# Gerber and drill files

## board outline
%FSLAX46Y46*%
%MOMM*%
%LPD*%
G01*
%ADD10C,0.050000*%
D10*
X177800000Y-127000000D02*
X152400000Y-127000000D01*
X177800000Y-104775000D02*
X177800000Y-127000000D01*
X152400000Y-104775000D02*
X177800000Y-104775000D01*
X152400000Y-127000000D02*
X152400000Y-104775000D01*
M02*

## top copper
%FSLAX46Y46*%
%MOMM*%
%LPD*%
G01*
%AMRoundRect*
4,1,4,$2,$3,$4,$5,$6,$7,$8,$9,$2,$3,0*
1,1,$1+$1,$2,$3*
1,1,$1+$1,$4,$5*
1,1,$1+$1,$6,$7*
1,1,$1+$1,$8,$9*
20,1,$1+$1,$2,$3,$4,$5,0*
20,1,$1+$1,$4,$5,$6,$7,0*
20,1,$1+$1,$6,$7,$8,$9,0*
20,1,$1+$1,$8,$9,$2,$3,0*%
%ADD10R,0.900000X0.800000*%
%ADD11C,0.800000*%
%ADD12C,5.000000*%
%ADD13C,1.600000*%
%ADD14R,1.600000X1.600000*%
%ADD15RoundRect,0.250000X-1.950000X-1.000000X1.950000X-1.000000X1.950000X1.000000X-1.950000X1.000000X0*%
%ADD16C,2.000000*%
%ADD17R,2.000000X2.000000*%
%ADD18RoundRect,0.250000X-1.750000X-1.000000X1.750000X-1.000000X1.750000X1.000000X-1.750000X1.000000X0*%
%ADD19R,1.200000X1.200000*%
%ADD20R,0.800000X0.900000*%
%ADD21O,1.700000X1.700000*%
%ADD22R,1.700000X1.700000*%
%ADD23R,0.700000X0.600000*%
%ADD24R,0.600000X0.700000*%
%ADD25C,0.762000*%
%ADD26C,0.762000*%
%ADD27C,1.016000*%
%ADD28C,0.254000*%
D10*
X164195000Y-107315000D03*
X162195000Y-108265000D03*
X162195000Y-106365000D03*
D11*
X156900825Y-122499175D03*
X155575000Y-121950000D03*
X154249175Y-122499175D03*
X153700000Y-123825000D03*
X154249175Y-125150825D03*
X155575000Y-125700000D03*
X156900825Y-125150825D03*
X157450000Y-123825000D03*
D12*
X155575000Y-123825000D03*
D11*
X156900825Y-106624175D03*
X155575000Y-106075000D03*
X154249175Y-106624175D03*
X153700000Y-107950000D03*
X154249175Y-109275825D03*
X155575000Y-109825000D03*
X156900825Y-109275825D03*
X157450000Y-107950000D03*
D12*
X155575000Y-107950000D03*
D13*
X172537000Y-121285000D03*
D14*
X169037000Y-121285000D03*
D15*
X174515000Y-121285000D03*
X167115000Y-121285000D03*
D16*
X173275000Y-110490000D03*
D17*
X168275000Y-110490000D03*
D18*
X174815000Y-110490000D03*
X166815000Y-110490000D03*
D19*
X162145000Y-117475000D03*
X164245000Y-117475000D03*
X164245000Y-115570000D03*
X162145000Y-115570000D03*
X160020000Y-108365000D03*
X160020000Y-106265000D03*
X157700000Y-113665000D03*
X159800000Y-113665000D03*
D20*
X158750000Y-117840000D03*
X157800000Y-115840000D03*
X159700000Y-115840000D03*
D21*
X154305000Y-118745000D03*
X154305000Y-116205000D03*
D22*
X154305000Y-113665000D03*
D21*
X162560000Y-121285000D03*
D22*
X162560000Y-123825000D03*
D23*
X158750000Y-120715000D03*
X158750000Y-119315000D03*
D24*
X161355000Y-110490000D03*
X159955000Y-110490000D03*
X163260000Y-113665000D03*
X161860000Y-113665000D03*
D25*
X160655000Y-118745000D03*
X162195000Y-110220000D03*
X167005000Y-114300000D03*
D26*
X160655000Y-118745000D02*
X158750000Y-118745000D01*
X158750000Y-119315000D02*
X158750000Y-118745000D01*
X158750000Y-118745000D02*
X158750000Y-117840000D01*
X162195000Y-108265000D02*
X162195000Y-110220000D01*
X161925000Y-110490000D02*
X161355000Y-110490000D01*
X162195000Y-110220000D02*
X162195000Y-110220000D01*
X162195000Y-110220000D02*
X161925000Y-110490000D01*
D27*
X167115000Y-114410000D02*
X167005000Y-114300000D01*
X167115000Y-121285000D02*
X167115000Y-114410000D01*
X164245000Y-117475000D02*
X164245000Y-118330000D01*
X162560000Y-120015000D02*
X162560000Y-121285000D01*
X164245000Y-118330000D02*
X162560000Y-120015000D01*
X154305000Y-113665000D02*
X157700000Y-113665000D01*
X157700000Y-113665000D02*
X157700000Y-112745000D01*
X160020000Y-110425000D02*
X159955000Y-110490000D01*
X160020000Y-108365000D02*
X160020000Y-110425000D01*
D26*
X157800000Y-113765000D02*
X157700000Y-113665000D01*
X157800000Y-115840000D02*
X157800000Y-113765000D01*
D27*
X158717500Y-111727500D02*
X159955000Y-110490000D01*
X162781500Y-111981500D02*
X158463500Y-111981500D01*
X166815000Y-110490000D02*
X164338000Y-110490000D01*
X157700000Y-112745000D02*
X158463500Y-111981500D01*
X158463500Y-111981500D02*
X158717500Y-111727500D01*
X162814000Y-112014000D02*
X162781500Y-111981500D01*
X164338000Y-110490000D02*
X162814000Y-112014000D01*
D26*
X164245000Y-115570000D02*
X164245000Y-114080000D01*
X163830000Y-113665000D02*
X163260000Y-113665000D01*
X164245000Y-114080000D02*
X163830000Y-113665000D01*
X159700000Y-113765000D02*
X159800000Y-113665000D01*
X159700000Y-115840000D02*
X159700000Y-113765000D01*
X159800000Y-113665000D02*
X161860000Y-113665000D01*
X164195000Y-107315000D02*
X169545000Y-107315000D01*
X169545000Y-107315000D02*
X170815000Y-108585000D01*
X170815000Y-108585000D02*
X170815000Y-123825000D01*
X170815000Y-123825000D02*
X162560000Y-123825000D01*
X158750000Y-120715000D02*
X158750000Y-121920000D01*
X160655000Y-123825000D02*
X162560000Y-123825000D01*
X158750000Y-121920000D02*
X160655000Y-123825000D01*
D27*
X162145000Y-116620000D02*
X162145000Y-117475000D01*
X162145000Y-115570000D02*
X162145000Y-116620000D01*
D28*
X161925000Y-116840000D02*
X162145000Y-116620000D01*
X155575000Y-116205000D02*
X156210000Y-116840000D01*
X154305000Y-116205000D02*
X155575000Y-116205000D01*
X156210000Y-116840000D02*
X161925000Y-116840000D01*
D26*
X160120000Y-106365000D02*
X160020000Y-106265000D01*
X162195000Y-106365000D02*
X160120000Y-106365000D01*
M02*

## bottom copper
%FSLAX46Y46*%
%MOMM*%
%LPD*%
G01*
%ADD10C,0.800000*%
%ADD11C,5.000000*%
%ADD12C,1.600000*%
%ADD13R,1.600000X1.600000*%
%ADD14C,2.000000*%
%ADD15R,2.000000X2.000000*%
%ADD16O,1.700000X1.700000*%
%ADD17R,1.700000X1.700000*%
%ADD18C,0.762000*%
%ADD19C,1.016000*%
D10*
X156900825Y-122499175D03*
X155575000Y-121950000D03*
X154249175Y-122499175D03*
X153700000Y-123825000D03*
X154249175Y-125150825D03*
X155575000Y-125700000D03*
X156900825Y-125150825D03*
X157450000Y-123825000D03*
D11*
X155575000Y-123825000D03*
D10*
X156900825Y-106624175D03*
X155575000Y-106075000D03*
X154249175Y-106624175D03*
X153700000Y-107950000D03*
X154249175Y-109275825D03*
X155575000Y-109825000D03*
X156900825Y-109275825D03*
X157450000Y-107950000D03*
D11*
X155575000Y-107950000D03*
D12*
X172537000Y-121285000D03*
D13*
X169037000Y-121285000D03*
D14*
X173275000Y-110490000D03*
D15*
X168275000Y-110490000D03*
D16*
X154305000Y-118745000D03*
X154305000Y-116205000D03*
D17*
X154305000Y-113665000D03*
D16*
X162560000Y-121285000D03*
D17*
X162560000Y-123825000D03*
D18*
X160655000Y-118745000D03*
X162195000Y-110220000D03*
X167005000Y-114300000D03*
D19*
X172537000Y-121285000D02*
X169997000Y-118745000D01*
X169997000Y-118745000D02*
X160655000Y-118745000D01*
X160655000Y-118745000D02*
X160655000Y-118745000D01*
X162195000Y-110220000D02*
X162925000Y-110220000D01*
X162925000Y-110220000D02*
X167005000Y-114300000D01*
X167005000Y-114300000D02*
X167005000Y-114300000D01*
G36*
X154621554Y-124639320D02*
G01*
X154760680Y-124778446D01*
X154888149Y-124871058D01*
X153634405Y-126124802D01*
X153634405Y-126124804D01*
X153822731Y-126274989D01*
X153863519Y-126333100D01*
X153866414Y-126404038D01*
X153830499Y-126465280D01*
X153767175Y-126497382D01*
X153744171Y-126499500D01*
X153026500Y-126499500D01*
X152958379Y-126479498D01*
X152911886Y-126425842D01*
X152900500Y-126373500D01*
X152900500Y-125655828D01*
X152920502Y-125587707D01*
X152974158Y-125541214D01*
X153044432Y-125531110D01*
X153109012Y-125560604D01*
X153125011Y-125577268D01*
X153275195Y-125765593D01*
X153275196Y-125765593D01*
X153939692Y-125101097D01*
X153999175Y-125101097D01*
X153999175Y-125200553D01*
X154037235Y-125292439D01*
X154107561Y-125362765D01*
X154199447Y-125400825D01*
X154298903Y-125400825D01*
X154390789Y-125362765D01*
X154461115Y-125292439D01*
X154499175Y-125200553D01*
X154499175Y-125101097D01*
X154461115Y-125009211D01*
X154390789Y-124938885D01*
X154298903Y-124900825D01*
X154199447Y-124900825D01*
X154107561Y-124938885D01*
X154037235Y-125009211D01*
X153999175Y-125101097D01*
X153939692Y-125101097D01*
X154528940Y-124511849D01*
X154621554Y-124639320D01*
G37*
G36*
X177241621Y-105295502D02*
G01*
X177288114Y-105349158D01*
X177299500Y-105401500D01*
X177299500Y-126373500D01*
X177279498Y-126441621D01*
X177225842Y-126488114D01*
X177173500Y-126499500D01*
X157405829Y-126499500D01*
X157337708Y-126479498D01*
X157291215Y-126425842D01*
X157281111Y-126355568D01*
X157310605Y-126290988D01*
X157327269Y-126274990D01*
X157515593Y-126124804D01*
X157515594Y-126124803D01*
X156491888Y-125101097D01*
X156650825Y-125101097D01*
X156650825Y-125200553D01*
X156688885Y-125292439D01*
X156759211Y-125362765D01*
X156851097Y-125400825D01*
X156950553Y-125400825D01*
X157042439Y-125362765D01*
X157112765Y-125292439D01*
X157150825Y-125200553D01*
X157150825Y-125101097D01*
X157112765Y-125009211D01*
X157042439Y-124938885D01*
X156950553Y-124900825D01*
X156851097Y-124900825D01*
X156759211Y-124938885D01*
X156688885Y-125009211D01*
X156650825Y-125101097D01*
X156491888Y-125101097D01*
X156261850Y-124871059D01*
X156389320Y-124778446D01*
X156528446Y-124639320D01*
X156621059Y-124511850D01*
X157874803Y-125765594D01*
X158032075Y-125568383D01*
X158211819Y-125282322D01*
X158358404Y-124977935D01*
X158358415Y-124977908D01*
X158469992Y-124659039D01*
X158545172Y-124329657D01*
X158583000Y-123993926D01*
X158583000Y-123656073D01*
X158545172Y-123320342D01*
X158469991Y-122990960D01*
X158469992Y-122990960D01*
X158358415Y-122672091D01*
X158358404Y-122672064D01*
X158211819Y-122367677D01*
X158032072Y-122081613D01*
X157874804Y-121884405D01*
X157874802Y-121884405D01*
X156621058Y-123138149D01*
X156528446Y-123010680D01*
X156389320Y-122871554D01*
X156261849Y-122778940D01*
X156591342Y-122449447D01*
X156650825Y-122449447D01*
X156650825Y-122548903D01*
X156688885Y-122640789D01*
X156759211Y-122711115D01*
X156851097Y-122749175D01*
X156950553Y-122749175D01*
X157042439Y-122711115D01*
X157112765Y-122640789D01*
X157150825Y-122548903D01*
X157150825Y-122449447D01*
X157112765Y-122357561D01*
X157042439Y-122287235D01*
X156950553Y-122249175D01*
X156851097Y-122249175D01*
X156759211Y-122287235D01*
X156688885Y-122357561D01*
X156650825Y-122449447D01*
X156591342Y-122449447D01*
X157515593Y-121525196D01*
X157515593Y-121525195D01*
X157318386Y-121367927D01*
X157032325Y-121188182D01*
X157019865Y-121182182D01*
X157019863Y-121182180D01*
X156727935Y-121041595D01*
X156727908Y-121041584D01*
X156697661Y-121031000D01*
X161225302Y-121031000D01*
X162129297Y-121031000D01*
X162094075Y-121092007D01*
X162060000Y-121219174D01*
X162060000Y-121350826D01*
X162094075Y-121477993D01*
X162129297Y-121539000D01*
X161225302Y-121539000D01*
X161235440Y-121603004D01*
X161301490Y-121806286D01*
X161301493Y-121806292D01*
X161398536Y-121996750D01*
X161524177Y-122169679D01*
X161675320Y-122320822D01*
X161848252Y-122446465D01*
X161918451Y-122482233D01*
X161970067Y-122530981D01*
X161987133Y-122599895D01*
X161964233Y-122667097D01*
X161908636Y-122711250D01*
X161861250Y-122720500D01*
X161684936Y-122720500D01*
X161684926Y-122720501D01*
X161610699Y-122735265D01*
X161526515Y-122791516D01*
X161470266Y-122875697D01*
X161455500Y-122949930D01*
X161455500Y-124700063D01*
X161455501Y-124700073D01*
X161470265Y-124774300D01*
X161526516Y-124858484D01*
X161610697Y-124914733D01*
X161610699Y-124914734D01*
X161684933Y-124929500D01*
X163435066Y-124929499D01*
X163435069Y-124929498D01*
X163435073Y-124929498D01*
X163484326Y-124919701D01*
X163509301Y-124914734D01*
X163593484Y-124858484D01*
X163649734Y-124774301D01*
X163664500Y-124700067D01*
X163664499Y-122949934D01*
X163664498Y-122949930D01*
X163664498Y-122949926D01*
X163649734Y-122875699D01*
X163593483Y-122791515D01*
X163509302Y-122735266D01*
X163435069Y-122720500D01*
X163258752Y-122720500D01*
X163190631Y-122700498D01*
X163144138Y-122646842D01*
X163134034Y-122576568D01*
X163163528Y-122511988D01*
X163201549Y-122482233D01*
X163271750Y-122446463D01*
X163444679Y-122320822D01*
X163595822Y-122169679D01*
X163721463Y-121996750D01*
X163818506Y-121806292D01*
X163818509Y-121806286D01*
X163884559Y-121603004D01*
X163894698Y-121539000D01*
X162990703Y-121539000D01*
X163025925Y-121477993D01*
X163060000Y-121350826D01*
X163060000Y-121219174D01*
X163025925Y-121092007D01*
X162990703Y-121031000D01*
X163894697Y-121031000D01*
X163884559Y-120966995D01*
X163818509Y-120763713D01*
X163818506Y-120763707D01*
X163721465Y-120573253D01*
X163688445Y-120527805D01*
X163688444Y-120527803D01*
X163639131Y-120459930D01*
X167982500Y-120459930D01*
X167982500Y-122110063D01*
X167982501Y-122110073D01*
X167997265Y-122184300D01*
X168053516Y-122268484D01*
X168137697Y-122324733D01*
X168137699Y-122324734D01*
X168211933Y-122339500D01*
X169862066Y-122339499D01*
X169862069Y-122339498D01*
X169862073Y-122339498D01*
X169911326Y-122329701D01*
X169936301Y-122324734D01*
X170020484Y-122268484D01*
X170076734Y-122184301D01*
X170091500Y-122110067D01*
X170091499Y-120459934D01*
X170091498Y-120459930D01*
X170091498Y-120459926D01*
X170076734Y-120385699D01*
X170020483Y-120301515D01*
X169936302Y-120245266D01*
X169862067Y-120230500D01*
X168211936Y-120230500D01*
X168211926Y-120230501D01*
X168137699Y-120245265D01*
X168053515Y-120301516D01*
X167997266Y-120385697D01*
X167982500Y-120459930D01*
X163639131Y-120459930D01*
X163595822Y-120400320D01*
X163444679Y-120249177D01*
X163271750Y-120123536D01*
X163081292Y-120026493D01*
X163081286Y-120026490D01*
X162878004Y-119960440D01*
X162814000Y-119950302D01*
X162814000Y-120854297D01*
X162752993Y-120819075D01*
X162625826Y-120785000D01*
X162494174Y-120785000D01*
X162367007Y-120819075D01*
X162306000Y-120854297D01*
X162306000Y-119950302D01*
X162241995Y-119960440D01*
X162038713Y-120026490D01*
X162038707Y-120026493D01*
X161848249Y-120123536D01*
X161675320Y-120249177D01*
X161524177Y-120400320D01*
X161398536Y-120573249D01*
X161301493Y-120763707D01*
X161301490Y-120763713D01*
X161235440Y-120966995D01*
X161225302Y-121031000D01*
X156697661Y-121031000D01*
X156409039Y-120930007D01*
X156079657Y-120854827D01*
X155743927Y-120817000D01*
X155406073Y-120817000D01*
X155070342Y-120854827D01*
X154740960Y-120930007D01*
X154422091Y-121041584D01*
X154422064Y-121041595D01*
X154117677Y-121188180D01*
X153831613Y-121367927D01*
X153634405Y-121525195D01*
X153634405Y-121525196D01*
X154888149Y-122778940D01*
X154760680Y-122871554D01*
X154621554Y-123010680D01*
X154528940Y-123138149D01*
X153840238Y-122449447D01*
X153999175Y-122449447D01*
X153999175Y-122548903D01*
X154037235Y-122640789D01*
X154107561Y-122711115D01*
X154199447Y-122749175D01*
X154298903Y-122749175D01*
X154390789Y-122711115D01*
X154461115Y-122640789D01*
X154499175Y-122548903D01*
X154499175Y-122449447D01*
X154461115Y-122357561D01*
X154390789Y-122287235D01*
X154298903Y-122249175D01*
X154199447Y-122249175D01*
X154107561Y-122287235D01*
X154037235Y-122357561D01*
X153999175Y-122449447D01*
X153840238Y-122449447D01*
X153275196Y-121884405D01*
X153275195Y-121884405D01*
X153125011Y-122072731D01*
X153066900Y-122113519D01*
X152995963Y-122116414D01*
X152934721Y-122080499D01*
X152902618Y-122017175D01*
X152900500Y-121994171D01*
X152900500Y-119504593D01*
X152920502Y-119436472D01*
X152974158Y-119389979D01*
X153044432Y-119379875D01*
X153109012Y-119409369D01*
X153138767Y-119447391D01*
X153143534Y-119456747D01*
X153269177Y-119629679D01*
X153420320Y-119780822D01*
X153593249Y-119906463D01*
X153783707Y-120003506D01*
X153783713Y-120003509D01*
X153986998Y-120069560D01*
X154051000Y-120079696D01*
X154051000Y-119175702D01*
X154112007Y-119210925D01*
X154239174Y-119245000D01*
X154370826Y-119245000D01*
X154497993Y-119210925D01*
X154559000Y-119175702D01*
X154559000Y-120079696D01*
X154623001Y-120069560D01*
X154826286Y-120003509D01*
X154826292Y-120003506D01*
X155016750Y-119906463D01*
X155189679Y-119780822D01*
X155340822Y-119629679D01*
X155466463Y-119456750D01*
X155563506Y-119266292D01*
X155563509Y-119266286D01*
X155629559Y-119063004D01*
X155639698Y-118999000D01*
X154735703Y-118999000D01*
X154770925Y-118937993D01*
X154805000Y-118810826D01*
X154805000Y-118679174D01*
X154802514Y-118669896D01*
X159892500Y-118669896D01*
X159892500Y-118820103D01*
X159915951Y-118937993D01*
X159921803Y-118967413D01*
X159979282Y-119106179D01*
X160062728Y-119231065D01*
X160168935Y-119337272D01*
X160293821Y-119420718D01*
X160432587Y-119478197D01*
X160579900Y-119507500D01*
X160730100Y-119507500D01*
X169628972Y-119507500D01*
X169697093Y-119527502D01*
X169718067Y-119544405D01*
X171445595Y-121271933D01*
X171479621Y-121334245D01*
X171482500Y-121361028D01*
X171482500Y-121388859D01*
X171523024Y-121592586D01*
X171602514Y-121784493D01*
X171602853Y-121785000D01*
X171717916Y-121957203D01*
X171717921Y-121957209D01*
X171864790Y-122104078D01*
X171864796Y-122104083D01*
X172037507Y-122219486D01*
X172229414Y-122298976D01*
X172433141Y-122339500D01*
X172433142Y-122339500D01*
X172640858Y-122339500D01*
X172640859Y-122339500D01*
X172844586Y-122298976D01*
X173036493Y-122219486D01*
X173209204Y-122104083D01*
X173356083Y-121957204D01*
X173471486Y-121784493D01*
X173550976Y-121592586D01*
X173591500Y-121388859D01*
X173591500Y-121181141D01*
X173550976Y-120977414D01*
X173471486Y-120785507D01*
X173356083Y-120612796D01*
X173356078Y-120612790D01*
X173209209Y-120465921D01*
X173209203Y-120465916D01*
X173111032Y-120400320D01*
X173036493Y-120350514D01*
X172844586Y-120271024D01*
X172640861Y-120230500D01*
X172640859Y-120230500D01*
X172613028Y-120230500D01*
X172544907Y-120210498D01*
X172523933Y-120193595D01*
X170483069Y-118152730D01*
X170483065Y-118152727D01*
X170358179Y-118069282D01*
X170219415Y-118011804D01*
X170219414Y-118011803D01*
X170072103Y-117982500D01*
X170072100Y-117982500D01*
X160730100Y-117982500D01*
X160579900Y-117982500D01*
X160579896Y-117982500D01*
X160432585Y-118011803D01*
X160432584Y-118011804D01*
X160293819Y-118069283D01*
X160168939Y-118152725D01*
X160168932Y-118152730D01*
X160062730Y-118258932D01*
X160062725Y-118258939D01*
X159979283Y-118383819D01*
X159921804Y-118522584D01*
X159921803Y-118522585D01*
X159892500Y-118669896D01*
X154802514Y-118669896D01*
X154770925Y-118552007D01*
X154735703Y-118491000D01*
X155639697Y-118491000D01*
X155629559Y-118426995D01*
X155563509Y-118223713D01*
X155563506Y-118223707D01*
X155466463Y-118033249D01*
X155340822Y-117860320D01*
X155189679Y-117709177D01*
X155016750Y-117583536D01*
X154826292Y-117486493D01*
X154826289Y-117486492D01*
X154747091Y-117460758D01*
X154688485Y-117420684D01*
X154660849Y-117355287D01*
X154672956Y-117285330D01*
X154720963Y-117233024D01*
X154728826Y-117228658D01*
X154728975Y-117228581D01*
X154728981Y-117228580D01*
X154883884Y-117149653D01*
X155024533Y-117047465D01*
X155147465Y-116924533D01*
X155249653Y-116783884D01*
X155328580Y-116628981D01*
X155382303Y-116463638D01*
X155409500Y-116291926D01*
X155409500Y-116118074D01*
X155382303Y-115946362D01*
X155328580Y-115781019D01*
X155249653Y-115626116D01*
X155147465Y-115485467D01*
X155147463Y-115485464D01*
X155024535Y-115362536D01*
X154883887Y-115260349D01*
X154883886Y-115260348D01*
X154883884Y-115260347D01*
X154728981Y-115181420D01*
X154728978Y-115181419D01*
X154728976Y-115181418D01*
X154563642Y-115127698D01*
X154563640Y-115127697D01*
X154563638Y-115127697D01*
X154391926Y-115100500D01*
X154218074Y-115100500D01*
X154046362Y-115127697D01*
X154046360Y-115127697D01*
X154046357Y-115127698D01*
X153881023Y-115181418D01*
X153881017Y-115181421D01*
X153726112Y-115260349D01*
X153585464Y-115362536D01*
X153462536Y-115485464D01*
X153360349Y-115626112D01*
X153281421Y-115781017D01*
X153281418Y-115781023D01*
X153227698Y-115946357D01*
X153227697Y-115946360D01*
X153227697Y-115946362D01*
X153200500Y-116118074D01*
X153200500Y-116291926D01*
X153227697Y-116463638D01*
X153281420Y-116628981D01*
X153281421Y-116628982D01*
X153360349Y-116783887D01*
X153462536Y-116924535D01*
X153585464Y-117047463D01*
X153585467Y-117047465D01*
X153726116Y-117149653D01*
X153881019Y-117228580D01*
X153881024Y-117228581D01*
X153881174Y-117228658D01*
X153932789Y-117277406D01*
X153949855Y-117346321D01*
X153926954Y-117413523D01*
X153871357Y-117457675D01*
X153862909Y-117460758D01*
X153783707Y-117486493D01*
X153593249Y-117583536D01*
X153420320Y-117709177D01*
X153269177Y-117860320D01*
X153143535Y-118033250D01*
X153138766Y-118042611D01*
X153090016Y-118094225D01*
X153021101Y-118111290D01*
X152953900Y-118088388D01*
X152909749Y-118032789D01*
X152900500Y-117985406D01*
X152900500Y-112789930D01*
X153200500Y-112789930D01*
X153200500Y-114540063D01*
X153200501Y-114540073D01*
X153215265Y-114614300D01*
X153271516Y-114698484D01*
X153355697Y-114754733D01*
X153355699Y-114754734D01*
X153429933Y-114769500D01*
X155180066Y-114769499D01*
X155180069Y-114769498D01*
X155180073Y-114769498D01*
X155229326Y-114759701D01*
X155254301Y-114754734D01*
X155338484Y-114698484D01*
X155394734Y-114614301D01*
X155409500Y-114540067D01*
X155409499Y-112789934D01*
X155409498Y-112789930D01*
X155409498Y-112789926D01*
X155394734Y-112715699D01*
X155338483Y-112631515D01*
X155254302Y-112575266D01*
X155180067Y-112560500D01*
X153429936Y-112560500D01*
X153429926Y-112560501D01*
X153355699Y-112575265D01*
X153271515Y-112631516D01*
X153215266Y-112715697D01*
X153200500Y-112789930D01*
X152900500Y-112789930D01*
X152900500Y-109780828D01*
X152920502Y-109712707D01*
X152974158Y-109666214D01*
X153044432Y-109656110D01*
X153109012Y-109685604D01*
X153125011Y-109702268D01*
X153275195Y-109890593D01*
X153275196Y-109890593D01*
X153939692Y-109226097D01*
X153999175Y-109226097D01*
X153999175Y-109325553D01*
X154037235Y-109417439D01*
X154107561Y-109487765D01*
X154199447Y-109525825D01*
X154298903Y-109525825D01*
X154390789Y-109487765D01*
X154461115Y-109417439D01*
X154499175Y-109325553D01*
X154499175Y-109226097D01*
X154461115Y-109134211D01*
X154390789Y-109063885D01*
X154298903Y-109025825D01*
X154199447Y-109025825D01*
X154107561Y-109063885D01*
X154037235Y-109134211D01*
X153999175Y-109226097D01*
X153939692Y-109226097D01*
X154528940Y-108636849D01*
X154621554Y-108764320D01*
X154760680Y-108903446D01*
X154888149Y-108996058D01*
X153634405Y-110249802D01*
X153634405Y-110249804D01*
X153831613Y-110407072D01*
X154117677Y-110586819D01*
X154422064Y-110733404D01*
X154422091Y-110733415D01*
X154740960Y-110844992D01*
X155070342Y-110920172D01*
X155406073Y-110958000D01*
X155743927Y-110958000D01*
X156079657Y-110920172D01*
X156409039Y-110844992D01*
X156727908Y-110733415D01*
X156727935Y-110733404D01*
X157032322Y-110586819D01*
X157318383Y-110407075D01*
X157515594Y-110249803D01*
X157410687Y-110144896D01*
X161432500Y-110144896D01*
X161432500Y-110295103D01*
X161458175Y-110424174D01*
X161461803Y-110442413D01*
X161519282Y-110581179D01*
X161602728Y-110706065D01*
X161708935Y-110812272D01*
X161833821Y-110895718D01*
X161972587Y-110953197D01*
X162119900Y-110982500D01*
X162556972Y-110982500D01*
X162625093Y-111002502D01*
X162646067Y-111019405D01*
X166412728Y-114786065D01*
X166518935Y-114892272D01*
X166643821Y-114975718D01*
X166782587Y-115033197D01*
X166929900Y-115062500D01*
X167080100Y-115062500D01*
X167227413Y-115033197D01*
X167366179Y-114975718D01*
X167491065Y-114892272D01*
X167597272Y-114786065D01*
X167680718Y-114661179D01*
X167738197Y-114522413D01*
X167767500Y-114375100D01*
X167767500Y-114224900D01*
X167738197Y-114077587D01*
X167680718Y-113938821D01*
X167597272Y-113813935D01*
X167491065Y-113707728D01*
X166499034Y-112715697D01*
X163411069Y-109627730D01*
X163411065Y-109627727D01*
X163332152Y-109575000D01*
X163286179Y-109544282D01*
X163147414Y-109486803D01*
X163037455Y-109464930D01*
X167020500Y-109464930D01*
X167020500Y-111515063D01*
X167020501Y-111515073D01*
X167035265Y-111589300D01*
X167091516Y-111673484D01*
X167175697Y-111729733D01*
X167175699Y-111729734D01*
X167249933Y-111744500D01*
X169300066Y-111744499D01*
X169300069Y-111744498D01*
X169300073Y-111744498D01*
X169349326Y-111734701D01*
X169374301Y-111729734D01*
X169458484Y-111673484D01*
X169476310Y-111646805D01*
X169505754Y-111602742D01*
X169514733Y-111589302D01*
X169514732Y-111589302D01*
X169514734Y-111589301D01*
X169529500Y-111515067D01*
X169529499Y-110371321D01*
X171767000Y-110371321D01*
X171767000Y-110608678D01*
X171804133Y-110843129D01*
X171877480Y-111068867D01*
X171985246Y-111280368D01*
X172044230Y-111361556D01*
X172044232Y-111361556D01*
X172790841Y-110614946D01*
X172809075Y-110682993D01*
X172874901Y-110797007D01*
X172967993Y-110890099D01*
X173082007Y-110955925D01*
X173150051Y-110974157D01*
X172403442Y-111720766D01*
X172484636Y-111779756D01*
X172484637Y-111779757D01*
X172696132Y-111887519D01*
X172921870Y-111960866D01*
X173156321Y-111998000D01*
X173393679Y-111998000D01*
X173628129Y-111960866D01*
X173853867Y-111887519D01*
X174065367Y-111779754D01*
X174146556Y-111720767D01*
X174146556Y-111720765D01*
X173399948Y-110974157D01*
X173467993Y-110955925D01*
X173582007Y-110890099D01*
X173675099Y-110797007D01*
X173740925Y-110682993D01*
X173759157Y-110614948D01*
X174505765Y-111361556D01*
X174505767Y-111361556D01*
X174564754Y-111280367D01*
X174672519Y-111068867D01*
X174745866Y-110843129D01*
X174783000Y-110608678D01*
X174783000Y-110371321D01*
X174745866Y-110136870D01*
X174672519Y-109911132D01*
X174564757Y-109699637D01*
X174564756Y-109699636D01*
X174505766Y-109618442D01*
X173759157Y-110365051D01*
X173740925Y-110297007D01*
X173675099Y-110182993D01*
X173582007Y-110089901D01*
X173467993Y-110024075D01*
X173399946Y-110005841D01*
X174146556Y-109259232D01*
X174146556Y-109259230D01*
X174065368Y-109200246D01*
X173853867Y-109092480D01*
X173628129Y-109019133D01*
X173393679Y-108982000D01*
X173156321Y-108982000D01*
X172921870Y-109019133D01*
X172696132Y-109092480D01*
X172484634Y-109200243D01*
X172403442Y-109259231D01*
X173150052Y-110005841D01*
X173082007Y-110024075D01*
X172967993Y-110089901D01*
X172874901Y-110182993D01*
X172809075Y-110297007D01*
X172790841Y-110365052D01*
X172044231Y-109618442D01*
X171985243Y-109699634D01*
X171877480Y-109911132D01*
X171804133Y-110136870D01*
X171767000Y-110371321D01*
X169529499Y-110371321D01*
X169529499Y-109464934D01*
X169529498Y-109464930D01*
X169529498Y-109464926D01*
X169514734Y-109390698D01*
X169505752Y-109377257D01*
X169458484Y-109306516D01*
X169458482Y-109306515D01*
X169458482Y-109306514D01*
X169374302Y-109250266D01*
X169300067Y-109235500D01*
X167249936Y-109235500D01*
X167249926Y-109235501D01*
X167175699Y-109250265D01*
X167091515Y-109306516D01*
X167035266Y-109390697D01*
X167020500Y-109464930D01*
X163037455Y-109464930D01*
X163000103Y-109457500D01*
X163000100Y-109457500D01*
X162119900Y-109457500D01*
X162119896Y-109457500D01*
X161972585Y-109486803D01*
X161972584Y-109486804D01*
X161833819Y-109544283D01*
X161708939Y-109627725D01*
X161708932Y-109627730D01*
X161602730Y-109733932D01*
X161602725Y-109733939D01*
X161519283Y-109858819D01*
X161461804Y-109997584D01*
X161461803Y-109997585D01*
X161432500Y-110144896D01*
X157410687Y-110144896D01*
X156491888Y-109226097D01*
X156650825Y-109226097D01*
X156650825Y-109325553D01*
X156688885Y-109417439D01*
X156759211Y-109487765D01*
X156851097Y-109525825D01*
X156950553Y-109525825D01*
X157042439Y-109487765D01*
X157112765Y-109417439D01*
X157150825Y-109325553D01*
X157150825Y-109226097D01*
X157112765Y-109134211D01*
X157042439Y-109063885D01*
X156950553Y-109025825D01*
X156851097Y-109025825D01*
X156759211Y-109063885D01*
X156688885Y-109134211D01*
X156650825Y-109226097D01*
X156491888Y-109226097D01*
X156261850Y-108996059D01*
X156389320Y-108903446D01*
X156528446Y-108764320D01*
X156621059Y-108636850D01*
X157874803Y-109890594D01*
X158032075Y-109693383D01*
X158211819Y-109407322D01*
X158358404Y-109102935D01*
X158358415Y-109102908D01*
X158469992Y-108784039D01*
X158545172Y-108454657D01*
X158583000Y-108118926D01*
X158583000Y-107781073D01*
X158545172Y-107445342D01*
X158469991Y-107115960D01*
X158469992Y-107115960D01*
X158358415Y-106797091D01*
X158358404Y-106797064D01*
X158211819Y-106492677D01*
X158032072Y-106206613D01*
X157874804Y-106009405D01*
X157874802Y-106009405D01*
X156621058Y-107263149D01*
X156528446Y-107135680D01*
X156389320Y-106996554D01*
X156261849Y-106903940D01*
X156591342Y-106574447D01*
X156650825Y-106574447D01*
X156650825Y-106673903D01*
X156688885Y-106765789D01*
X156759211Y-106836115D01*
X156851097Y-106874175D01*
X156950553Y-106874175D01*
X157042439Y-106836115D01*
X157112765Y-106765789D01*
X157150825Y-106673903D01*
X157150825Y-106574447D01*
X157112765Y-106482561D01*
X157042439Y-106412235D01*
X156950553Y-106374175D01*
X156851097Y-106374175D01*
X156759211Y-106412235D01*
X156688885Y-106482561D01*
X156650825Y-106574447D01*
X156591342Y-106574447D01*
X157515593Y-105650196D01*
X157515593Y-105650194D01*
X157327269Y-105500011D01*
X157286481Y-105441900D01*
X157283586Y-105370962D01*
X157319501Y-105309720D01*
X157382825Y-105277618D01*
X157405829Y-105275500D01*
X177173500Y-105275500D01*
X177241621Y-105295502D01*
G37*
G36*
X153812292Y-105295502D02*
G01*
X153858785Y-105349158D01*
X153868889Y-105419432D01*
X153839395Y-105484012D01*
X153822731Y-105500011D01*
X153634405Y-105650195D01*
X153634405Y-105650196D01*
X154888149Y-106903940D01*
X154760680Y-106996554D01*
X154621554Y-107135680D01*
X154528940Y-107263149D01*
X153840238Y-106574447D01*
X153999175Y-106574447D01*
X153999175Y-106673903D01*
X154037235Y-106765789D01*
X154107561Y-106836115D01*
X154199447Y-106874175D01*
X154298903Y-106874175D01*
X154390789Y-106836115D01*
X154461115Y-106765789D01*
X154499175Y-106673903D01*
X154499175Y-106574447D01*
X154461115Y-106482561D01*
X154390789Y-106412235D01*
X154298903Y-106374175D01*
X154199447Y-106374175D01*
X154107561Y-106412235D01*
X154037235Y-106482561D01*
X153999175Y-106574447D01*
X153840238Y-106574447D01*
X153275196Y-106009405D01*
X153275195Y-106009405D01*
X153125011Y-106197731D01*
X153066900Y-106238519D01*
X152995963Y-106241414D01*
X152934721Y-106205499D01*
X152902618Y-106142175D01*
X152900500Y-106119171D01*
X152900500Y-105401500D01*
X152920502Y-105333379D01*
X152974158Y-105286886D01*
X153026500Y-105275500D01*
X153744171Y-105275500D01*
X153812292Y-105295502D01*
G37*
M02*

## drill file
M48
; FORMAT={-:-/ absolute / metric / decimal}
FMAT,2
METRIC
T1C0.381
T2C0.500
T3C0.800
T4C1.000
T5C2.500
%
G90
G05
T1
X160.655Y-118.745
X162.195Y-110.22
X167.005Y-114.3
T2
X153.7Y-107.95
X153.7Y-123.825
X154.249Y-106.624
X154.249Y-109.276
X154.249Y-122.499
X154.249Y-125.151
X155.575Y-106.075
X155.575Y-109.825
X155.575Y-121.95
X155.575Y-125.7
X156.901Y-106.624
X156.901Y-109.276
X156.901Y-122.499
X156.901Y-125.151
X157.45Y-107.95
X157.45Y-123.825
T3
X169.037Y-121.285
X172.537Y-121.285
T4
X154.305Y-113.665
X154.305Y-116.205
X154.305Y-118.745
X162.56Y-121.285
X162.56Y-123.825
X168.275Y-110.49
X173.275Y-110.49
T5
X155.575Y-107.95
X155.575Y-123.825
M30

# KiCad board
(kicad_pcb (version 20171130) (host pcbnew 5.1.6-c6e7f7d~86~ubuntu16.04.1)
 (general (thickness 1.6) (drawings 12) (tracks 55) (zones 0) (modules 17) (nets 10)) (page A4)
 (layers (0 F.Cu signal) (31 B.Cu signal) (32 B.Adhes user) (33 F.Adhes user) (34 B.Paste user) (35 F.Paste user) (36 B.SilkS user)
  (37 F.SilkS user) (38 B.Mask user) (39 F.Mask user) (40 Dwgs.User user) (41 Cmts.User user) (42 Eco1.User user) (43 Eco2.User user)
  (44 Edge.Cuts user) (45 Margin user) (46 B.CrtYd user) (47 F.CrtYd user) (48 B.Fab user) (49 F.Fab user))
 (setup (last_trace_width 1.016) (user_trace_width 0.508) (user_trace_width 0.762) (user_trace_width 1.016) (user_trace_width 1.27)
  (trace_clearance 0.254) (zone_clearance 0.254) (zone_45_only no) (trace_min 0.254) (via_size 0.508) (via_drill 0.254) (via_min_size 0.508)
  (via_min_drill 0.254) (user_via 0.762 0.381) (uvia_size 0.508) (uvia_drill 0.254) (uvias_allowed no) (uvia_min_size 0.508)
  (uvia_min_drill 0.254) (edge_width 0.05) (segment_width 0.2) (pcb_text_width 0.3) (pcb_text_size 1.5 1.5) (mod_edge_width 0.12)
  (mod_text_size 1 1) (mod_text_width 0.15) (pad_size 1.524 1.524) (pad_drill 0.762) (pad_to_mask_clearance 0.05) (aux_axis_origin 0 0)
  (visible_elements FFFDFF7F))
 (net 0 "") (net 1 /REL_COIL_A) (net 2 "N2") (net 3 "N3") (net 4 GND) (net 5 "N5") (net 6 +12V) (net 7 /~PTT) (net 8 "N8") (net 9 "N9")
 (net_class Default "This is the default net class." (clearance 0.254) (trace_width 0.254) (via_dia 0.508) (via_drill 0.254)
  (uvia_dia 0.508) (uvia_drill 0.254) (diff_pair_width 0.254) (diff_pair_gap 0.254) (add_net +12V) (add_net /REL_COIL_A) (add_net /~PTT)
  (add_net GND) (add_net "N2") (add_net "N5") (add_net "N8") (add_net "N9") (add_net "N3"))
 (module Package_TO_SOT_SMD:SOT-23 (layer F.Cu) (at 163.195 107.315)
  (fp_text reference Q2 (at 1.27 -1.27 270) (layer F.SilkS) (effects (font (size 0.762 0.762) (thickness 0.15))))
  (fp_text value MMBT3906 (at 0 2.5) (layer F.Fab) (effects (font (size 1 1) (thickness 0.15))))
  (pad 3 smd rect (at 1 0) (size 0.9 0.8) (layers F.Cu F.Paste F.Mask) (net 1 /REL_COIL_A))
  (pad 2 smd rect (at -1 0.95) (size 0.9 0.8) (layers F.Cu F.Paste F.Mask) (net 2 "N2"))
  (pad 1 smd rect (at -1 -0.95) (size 0.9 0.8) (layers F.Cu F.Paste F.Mask) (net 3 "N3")))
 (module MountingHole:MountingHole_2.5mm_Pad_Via (layer F.Cu) (at 155.575 123.825)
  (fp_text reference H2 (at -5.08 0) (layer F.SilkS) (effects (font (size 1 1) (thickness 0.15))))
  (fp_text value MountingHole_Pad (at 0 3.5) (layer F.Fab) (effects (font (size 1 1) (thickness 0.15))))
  (pad 1 thru_hole circle (at 1.325825 -1.325825) (size 0.8 0.8) (drill 0.5) (layers *.Cu *.Mask) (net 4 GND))
  (pad 1 thru_hole circle (at 0 -1.875) (size 0.8 0.8) (drill 0.5) (layers *.Cu *.Mask) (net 4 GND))
  (pad 1 thru_hole circle (at -1.325825 -1.325825) (size 0.8 0.8) (drill 0.5) (layers *.Cu *.Mask) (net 4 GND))
  (pad 1 thru_hole circle (at -1.875 0) (size 0.8 0.8) (drill 0.5) (layers *.Cu *.Mask) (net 4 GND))
  (pad 1 thru_hole circle (at -1.325825 1.325825) (size 0.8 0.8) (drill 0.5) (layers *.Cu *.Mask) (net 4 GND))
  (pad 1 thru_hole circle (at 0 1.875) (size 0.8 0.8) (drill 0.5) (layers *.Cu *.Mask) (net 4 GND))
  (pad 1 thru_hole circle (at 1.325825 1.325825) (size 0.8 0.8) (drill 0.5) (layers *.Cu *.Mask) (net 4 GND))
  (pad 1 thru_hole circle (at 1.875 0) (size 0.8 0.8) (drill 0.5) (layers *.Cu *.Mask) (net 4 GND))
  (pad 1 thru_hole circle (at 0 0) (size 5 5) (drill 2.5) (layers *.Cu *.Mask) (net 4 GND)))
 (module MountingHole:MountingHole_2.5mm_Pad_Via (layer F.Cu) (at 155.575 107.95)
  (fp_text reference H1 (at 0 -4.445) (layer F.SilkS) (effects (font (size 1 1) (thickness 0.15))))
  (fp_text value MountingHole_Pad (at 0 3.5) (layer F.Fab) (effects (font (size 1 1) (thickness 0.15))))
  (pad 1 thru_hole circle (at 1.325825 -1.325825) (size 0.8 0.8) (drill 0.5) (layers *.Cu *.Mask) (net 4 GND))
  (pad 1 thru_hole circle (at 0 -1.875) (size 0.8 0.8) (drill 0.5) (layers *.Cu *.Mask) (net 4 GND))
  (pad 1 thru_hole circle (at -1.325825 -1.325825) (size 0.8 0.8) (drill 0.5) (layers *.Cu *.Mask) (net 4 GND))
  (pad 1 thru_hole circle (at -1.875 0) (size 0.8 0.8) (drill 0.5) (layers *.Cu *.Mask) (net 4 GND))
  (pad 1 thru_hole circle (at -1.325825 1.325825) (size 0.8 0.8) (drill 0.5) (layers *.Cu *.Mask) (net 4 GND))
  (pad 1 thru_hole circle (at 0 1.875) (size 0.8 0.8) (drill 0.5) (layers *.Cu *.Mask) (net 4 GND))
  (pad 1 thru_hole circle (at 1.325825 1.325825) (size 0.8 0.8) (drill 0.5) (layers *.Cu *.Mask) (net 4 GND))
  (pad 1 thru_hole circle (at 1.875 0) (size 0.8 0.8) (drill 0.5) (layers *.Cu *.Mask) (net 4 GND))
  (pad 1 thru_hole circle (at 0 0) (size 5 5) (drill 2.5) (layers *.Cu *.Mask) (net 4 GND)))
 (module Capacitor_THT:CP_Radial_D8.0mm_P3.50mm (layer F.Cu) (at 169.037 121.285)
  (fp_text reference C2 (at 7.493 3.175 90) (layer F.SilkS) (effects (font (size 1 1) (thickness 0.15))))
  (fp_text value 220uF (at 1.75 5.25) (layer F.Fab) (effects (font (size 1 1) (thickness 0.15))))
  (pad 2 thru_hole circle (at 3.5 0) (size 1.6 1.6) (drill 0.8) (layers *.Cu *.Mask) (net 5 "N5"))
  (pad 1 thru_hole rect (at 0 0) (size 1.6 1.6) (drill 0.8) (layers *.Cu *.Mask) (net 2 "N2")))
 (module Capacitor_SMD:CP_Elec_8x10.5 (layer F.Cu) (at 170.815 121.285)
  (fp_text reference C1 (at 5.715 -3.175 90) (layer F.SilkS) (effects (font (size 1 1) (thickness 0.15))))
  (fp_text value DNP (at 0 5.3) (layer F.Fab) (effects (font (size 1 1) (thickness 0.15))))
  (pad 2 smd roundrect (at 3.7 0) (size 4.4 2.5) (layers F.Cu F.Paste F.Mask) (roundrect_rratio 0.1) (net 5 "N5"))
  (pad 1 smd roundrect (at -3.7 0) (size 4.4 2.5) (layers F.Cu F.Paste F.Mask) (roundrect_rratio 0.1) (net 2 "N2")))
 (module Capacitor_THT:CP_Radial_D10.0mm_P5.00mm (layer F.Cu) (at 168.275 110.49)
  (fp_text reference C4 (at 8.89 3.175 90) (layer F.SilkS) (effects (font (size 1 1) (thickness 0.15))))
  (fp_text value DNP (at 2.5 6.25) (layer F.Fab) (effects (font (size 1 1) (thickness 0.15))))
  (pad 2 thru_hole circle (at 5 0) (size 2 2) (drill 1) (layers *.Cu *.Mask) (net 4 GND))
  (pad 1 thru_hole rect (at 0 0) (size 2 2) (drill 1) (layers *.Cu *.Mask) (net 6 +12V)))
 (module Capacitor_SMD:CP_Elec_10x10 (layer F.Cu) (at 170.815 110.49)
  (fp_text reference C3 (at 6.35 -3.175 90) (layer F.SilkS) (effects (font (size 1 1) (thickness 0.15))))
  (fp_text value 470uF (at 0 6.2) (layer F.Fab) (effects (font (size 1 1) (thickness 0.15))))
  (pad 2 smd roundrect (at 4 0) (size 4 2.5) (layers F.Cu F.Paste F.Mask) (roundrect_rratio 0.1) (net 4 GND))
  (pad 1 smd roundrect (at -4 0) (size 4 2.5) (layers F.Cu F.Paste F.Mask) (roundrect_rratio 0.1) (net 6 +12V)))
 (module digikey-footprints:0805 (layer F.Cu) (at 163.195 117.475)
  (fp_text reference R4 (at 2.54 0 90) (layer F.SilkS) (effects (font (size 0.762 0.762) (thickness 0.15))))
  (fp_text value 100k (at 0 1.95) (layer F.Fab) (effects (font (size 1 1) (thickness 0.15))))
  (pad 1 smd rect (at -1.05 0) (size 1.2 1.2) (layers F.Cu F.Paste F.Mask) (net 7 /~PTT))
  (pad 2 smd rect (at 1.05 0) (size 1.2 1.2) (layers F.Cu F.Paste F.Mask) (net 4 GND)))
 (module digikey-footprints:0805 (layer F.Cu) (at 163.195 115.57 180)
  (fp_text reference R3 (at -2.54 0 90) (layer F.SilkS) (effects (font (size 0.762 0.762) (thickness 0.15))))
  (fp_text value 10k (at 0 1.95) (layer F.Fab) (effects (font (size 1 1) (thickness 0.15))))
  (pad 1 smd rect (at -1.05 0 180) (size 1.2 1.2) (layers F.Cu F.Paste F.Mask) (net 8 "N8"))
  (pad 2 smd rect (at 1.05 0 180) (size 1.2 1.2) (layers F.Cu F.Paste F.Mask) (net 7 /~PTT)))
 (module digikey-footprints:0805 (layer F.Cu) (at 160.02 107.315 90)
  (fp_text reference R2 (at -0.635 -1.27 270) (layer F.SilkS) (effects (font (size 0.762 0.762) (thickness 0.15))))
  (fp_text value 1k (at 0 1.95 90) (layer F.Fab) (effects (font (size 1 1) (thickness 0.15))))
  (pad 1 smd rect (at -1.05 0 90) (size 1.2 1.2) (layers F.Cu F.Paste F.Mask) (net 6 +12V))
  (pad 2 smd rect (at 1.05 0 90) (size 1.2 1.2) (layers F.Cu F.Paste F.Mask) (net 3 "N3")))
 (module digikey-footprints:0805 (layer F.Cu) (at 158.75 113.665)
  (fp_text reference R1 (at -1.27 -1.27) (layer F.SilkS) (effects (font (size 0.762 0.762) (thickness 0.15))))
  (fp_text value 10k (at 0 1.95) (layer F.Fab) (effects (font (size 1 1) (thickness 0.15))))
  (pad 1 smd rect (at -1.05 0) (size 1.2 1.2) (layers F.Cu F.Paste F.Mask) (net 6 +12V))
  (pad 2 smd rect (at 1.05 0) (size 1.2 1.2) (layers F.Cu F.Paste F.Mask) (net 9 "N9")))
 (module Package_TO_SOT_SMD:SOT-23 (layer F.Cu) (at 158.75 116.84 270)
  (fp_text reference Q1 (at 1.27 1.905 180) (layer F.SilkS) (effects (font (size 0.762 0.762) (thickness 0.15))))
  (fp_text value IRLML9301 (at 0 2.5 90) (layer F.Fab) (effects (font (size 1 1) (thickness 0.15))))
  (pad 3 smd rect (at 1 0 270) (size 0.9 0.8) (layers F.Cu F.Paste F.Mask) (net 5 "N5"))
  (pad 2 smd rect (at -1 0.95 270) (size 0.9 0.8) (layers F.Cu F.Paste F.Mask) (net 6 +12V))
  (pad 1 smd rect (at -1 -0.95 270) (size 0.9 0.8) (layers F.Cu F.Paste F.Mask) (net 9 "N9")))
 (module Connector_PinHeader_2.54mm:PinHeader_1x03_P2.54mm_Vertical (layer F.Cu) (at 154.305 113.665)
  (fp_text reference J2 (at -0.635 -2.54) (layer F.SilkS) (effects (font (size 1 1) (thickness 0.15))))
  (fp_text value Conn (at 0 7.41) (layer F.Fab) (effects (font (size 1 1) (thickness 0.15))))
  (pad 3 thru_hole oval (at 0 5.08) (size 1.7 1.7) (drill 1) (layers *.Cu *.Mask) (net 4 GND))
  (pad 2 thru_hole oval (at 0 2.54) (size 1.7 1.7) (drill 1) (layers *.Cu *.Mask) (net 7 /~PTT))
  (pad 1 thru_hole rect (at 0 0) (size 1.7 1.7) (drill 1) (layers *.Cu *.Mask) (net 6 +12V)))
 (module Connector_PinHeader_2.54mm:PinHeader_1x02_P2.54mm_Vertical (layer F.Cu) (at 162.56 123.825 180)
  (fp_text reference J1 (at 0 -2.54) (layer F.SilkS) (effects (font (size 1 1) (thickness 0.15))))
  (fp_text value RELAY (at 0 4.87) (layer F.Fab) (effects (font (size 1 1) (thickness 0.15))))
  (pad 2 thru_hole oval (at 0 2.54 180) (size 1.7 1.7) (drill 1) (layers *.Cu *.Mask) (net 4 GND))
  (pad 1 thru_hole rect (at 0 0 180) (size 1.7 1.7) (drill 1) (layers *.Cu *.Mask) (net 1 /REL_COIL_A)))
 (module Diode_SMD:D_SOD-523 (layer F.Cu) (at 158.75 120.015 90)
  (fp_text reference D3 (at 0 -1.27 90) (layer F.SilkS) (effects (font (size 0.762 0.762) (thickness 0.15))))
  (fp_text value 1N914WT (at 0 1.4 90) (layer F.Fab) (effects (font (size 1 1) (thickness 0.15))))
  (pad 1 smd rect (at -0.7 0 270) (size 0.6 0.7) (layers F.Cu F.Paste F.Mask) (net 1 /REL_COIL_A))
  (pad 2 smd rect (at 0.7 0 270) (size 0.6 0.7) (layers F.Cu F.Paste F.Mask) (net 5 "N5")))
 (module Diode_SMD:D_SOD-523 (layer F.Cu) (at 160.655 110.49 180)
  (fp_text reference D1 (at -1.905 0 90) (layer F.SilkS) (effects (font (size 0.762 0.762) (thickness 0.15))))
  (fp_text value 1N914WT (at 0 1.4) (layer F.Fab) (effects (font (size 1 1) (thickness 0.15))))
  (pad 1 smd rect (at -0.7 0) (size 0.6 0.7) (layers F.Cu F.Paste F.Mask) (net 2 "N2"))
  (pad 2 smd rect (at 0.7 0) (size 0.6 0.7) (layers F.Cu F.Paste F.Mask) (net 6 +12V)))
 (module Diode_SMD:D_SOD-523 (layer F.Cu) (at 162.56 113.665 180)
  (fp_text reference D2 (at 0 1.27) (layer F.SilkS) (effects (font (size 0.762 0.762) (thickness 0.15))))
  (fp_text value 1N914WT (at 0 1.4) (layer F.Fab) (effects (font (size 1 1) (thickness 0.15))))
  (pad 1 smd rect (at -0.7 0) (size 0.6 0.7) (layers F.Cu F.Paste F.Mask) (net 8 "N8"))
  (pad 2 smd rect (at 0.7 0) (size 0.6 0.7) (layers F.Cu F.Paste F.Mask) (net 9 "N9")))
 (gr_line (start 177.8 127) (end 152.4 127) (layer Edge.Cuts) (width 0.05))
 (gr_line (start 177.8 104.775) (end 177.8 127) (layer Edge.Cuts) (width 0.05))
 (gr_line (start 152.4 104.775) (end 177.8 104.775) (layer Edge.Cuts) (width 0.05))
 (gr_line (start 152.4 127) (end 152.4 104.775) (layer Edge.Cuts) (width 0.05))
 (segment (start 172.537 121.285) (end 169.997 118.745) (width 1.016) (layer B.Cu) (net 5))
 (segment (start 169.997 118.745) (end 160.655 118.745) (width 1.016) (layer B.Cu) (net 5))
 (segment (start 160.655 118.745) (end 160.655 118.745) (width 1.016) (layer B.Cu) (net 5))
 (via (at 160.655 118.745) (size 0.762) (drill 0.381) (layers F.Cu B.Cu) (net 5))
 (segment (start 160.655 118.745) (end 158.75 118.745) (width 0.762) (layer F.Cu) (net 5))
 (segment (start 158.75 119.315) (end 158.75 118.745) (width 0.762) (layer F.Cu) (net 5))
 (segment (start 158.75 118.745) (end 158.75 117.84) (width 0.762) (layer F.Cu) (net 5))
 (segment (start 162.195 108.265) (end 162.195 110.22) (width 0.762) (layer F.Cu) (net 2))
 (segment (start 161.925 110.49) (end 161.355 110.49) (width 0.762) (layer F.Cu) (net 2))
 (segment (start 162.195 110.22) (end 162.195 110.22) (width 0.762) (layer F.Cu) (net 2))
 (segment (start 162.195 110.22) (end 161.925 110.49) (width 0.762) (layer F.Cu) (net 2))
 (via (at 162.195 110.22) (size 0.762) (drill 0.381) (layers F.Cu B.Cu) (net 2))
 (segment (start 162.195 110.22) (end 162.925 110.22) (width 1.016) (layer B.Cu) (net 2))
 (segment (start 162.925 110.22) (end 167.005 114.3) (width 1.016) (layer B.Cu) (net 2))
 (segment (start 167.005 114.3) (end 167.005 114.3) (width 1.016) (layer B.Cu) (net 2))
 (via (at 167.005 114.3) (size 0.762) (drill 0.381) (layers F.Cu B.Cu) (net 2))
 (segment (start 167.115 114.41) (end 167.005 114.3) (width 1.016) (layer F.Cu) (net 2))
 (segment (start 167.115 121.285) (end 167.115 114.41) (width 1.016) (layer F.Cu) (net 2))
 (segment (start 164.245 117.475) (end 164.245 118.33) (width 1.016) (layer F.Cu) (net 4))
 (segment (start 162.56 120.015) (end 162.56 121.285) (width 1.016) (layer F.Cu) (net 4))
 (segment (start 164.245 118.33) (end 162.56 120.015) (width 1.016) (layer F.Cu) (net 4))
 (segment (start 154.305 113.665) (end 157.7 113.665) (width 1.016) (layer F.Cu) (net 6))
 (segment (start 157.7 113.665) (end 157.7 112.745) (width 1.016) (layer F.Cu) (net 6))
 (segment (start 160.02 110.425) (end 159.955 110.49) (width 1.016) (layer F.Cu) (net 6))
 (segment (start 160.02 108.365) (end 160.02 110.425) (width 1.016) (layer F.Cu) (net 6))
 (segment (start 157.8 113.765) (end 157.7 113.665) (width 0.762) (layer F.Cu) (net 6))
 (segment (start 157.8 115.84) (end 157.8 113.765) (width 0.762) (layer F.Cu) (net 6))
 (segment (start 158.7175 111.7275) (end 159.955 110.49) (width 1.016) (layer F.Cu) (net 6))
 (segment (start 162.7815 111.9815) (end 158.4635 111.9815) (width 1.016) (layer F.Cu) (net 6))
 (segment (start 166.815 110.49) (end 164.338 110.49) (width 1.016) (layer F.Cu) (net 6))
 (segment (start 157.7 112.745) (end 158.4635 111.9815) (width 1.016) (layer F.Cu) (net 6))
 (segment (start 158.4635 111.9815) (end 158.7175 111.7275) (width 1.016) (layer F.Cu) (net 6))
 (segment (start 162.814 112.014) (end 162.7815 111.9815) (width 1.016) (layer F.Cu) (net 6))
 (segment (start 164.338 110.49) (end 162.814 112.014) (width 1.016) (layer F.Cu) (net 6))
 (segment (start 164.245 115.57) (end 164.245 114.08) (width 0.762) (layer F.Cu) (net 8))
 (segment (start 163.83 113.665) (end 163.26 113.665) (width 0.762) (layer F.Cu) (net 8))
 (segment (start 164.245 114.08) (end 163.83 113.665) (width 0.762) (layer F.Cu) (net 8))
 (segment (start 159.7 113.765) (end 159.8 113.665) (width 0.762) (layer F.Cu) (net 9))
 (segment (start 159.7 115.84) (end 159.7 113.765) (width 0.762) (layer F.Cu) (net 9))
 (segment (start 159.8 113.665) (end 161.86 113.665) (width 0.762) (layer F.Cu) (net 9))
 (segment (start 164.195 107.315) (end 169.545 107.315) (width 0.762) (layer F.Cu) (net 1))
 (segment (start 169.545 107.315) (end 170.815 108.585) (width 0.762) (layer F.Cu) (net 1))
 (segment (start 170.815 108.585) (end 170.815 123.825) (width 0.762) (layer F.Cu) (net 1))
 (segment (start 170.815 123.825) (end 162.56 123.825) (width 0.762) (layer F.Cu) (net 1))
 (segment (start 158.75 120.715) (end 158.75 121.92) (width 0.762) (layer F.Cu) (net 1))
 (segment (start 160.655 123.825) (end 162.56 123.825) (width 0.762) (layer F.Cu) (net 1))
 (segment (start 158.75 121.92) (end 160.655 123.825) (width 0.762) (layer F.Cu) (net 1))
 (segment (start 162.145 116.62) (end 162.145 117.475) (width 1.016) (layer F.Cu) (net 7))
 (segment (start 162.145 115.57) (end 162.145 116.62) (width 1.016) (layer F.Cu) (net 7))
 (segment (start 161.925 116.84) (end 162.145 116.62) (width 0.254) (layer F.Cu) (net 7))
 (segment (start 155.575 116.205) (end 156.21 116.84) (width 0.254) (layer F.Cu) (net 7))
 (segment (start 154.305 116.205) (end 155.575 116.205) (width 0.254) (layer F.Cu) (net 7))
 (segment (start 156.21 116.84) (end 161.925 116.84) (width 0.254) (layer F.Cu) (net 7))
 (segment (start 160.12 106.365) (end 160.02 106.265) (width 0.762) (layer F.Cu) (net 3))
 (segment (start 162.195 106.365) (end 160.12 106.365) (width 0.762) (layer F.Cu) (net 3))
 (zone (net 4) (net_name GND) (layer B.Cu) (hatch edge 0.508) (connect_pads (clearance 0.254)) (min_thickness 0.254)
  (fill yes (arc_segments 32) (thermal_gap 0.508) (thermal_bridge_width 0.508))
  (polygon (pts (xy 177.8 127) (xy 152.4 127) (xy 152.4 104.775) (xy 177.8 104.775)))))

